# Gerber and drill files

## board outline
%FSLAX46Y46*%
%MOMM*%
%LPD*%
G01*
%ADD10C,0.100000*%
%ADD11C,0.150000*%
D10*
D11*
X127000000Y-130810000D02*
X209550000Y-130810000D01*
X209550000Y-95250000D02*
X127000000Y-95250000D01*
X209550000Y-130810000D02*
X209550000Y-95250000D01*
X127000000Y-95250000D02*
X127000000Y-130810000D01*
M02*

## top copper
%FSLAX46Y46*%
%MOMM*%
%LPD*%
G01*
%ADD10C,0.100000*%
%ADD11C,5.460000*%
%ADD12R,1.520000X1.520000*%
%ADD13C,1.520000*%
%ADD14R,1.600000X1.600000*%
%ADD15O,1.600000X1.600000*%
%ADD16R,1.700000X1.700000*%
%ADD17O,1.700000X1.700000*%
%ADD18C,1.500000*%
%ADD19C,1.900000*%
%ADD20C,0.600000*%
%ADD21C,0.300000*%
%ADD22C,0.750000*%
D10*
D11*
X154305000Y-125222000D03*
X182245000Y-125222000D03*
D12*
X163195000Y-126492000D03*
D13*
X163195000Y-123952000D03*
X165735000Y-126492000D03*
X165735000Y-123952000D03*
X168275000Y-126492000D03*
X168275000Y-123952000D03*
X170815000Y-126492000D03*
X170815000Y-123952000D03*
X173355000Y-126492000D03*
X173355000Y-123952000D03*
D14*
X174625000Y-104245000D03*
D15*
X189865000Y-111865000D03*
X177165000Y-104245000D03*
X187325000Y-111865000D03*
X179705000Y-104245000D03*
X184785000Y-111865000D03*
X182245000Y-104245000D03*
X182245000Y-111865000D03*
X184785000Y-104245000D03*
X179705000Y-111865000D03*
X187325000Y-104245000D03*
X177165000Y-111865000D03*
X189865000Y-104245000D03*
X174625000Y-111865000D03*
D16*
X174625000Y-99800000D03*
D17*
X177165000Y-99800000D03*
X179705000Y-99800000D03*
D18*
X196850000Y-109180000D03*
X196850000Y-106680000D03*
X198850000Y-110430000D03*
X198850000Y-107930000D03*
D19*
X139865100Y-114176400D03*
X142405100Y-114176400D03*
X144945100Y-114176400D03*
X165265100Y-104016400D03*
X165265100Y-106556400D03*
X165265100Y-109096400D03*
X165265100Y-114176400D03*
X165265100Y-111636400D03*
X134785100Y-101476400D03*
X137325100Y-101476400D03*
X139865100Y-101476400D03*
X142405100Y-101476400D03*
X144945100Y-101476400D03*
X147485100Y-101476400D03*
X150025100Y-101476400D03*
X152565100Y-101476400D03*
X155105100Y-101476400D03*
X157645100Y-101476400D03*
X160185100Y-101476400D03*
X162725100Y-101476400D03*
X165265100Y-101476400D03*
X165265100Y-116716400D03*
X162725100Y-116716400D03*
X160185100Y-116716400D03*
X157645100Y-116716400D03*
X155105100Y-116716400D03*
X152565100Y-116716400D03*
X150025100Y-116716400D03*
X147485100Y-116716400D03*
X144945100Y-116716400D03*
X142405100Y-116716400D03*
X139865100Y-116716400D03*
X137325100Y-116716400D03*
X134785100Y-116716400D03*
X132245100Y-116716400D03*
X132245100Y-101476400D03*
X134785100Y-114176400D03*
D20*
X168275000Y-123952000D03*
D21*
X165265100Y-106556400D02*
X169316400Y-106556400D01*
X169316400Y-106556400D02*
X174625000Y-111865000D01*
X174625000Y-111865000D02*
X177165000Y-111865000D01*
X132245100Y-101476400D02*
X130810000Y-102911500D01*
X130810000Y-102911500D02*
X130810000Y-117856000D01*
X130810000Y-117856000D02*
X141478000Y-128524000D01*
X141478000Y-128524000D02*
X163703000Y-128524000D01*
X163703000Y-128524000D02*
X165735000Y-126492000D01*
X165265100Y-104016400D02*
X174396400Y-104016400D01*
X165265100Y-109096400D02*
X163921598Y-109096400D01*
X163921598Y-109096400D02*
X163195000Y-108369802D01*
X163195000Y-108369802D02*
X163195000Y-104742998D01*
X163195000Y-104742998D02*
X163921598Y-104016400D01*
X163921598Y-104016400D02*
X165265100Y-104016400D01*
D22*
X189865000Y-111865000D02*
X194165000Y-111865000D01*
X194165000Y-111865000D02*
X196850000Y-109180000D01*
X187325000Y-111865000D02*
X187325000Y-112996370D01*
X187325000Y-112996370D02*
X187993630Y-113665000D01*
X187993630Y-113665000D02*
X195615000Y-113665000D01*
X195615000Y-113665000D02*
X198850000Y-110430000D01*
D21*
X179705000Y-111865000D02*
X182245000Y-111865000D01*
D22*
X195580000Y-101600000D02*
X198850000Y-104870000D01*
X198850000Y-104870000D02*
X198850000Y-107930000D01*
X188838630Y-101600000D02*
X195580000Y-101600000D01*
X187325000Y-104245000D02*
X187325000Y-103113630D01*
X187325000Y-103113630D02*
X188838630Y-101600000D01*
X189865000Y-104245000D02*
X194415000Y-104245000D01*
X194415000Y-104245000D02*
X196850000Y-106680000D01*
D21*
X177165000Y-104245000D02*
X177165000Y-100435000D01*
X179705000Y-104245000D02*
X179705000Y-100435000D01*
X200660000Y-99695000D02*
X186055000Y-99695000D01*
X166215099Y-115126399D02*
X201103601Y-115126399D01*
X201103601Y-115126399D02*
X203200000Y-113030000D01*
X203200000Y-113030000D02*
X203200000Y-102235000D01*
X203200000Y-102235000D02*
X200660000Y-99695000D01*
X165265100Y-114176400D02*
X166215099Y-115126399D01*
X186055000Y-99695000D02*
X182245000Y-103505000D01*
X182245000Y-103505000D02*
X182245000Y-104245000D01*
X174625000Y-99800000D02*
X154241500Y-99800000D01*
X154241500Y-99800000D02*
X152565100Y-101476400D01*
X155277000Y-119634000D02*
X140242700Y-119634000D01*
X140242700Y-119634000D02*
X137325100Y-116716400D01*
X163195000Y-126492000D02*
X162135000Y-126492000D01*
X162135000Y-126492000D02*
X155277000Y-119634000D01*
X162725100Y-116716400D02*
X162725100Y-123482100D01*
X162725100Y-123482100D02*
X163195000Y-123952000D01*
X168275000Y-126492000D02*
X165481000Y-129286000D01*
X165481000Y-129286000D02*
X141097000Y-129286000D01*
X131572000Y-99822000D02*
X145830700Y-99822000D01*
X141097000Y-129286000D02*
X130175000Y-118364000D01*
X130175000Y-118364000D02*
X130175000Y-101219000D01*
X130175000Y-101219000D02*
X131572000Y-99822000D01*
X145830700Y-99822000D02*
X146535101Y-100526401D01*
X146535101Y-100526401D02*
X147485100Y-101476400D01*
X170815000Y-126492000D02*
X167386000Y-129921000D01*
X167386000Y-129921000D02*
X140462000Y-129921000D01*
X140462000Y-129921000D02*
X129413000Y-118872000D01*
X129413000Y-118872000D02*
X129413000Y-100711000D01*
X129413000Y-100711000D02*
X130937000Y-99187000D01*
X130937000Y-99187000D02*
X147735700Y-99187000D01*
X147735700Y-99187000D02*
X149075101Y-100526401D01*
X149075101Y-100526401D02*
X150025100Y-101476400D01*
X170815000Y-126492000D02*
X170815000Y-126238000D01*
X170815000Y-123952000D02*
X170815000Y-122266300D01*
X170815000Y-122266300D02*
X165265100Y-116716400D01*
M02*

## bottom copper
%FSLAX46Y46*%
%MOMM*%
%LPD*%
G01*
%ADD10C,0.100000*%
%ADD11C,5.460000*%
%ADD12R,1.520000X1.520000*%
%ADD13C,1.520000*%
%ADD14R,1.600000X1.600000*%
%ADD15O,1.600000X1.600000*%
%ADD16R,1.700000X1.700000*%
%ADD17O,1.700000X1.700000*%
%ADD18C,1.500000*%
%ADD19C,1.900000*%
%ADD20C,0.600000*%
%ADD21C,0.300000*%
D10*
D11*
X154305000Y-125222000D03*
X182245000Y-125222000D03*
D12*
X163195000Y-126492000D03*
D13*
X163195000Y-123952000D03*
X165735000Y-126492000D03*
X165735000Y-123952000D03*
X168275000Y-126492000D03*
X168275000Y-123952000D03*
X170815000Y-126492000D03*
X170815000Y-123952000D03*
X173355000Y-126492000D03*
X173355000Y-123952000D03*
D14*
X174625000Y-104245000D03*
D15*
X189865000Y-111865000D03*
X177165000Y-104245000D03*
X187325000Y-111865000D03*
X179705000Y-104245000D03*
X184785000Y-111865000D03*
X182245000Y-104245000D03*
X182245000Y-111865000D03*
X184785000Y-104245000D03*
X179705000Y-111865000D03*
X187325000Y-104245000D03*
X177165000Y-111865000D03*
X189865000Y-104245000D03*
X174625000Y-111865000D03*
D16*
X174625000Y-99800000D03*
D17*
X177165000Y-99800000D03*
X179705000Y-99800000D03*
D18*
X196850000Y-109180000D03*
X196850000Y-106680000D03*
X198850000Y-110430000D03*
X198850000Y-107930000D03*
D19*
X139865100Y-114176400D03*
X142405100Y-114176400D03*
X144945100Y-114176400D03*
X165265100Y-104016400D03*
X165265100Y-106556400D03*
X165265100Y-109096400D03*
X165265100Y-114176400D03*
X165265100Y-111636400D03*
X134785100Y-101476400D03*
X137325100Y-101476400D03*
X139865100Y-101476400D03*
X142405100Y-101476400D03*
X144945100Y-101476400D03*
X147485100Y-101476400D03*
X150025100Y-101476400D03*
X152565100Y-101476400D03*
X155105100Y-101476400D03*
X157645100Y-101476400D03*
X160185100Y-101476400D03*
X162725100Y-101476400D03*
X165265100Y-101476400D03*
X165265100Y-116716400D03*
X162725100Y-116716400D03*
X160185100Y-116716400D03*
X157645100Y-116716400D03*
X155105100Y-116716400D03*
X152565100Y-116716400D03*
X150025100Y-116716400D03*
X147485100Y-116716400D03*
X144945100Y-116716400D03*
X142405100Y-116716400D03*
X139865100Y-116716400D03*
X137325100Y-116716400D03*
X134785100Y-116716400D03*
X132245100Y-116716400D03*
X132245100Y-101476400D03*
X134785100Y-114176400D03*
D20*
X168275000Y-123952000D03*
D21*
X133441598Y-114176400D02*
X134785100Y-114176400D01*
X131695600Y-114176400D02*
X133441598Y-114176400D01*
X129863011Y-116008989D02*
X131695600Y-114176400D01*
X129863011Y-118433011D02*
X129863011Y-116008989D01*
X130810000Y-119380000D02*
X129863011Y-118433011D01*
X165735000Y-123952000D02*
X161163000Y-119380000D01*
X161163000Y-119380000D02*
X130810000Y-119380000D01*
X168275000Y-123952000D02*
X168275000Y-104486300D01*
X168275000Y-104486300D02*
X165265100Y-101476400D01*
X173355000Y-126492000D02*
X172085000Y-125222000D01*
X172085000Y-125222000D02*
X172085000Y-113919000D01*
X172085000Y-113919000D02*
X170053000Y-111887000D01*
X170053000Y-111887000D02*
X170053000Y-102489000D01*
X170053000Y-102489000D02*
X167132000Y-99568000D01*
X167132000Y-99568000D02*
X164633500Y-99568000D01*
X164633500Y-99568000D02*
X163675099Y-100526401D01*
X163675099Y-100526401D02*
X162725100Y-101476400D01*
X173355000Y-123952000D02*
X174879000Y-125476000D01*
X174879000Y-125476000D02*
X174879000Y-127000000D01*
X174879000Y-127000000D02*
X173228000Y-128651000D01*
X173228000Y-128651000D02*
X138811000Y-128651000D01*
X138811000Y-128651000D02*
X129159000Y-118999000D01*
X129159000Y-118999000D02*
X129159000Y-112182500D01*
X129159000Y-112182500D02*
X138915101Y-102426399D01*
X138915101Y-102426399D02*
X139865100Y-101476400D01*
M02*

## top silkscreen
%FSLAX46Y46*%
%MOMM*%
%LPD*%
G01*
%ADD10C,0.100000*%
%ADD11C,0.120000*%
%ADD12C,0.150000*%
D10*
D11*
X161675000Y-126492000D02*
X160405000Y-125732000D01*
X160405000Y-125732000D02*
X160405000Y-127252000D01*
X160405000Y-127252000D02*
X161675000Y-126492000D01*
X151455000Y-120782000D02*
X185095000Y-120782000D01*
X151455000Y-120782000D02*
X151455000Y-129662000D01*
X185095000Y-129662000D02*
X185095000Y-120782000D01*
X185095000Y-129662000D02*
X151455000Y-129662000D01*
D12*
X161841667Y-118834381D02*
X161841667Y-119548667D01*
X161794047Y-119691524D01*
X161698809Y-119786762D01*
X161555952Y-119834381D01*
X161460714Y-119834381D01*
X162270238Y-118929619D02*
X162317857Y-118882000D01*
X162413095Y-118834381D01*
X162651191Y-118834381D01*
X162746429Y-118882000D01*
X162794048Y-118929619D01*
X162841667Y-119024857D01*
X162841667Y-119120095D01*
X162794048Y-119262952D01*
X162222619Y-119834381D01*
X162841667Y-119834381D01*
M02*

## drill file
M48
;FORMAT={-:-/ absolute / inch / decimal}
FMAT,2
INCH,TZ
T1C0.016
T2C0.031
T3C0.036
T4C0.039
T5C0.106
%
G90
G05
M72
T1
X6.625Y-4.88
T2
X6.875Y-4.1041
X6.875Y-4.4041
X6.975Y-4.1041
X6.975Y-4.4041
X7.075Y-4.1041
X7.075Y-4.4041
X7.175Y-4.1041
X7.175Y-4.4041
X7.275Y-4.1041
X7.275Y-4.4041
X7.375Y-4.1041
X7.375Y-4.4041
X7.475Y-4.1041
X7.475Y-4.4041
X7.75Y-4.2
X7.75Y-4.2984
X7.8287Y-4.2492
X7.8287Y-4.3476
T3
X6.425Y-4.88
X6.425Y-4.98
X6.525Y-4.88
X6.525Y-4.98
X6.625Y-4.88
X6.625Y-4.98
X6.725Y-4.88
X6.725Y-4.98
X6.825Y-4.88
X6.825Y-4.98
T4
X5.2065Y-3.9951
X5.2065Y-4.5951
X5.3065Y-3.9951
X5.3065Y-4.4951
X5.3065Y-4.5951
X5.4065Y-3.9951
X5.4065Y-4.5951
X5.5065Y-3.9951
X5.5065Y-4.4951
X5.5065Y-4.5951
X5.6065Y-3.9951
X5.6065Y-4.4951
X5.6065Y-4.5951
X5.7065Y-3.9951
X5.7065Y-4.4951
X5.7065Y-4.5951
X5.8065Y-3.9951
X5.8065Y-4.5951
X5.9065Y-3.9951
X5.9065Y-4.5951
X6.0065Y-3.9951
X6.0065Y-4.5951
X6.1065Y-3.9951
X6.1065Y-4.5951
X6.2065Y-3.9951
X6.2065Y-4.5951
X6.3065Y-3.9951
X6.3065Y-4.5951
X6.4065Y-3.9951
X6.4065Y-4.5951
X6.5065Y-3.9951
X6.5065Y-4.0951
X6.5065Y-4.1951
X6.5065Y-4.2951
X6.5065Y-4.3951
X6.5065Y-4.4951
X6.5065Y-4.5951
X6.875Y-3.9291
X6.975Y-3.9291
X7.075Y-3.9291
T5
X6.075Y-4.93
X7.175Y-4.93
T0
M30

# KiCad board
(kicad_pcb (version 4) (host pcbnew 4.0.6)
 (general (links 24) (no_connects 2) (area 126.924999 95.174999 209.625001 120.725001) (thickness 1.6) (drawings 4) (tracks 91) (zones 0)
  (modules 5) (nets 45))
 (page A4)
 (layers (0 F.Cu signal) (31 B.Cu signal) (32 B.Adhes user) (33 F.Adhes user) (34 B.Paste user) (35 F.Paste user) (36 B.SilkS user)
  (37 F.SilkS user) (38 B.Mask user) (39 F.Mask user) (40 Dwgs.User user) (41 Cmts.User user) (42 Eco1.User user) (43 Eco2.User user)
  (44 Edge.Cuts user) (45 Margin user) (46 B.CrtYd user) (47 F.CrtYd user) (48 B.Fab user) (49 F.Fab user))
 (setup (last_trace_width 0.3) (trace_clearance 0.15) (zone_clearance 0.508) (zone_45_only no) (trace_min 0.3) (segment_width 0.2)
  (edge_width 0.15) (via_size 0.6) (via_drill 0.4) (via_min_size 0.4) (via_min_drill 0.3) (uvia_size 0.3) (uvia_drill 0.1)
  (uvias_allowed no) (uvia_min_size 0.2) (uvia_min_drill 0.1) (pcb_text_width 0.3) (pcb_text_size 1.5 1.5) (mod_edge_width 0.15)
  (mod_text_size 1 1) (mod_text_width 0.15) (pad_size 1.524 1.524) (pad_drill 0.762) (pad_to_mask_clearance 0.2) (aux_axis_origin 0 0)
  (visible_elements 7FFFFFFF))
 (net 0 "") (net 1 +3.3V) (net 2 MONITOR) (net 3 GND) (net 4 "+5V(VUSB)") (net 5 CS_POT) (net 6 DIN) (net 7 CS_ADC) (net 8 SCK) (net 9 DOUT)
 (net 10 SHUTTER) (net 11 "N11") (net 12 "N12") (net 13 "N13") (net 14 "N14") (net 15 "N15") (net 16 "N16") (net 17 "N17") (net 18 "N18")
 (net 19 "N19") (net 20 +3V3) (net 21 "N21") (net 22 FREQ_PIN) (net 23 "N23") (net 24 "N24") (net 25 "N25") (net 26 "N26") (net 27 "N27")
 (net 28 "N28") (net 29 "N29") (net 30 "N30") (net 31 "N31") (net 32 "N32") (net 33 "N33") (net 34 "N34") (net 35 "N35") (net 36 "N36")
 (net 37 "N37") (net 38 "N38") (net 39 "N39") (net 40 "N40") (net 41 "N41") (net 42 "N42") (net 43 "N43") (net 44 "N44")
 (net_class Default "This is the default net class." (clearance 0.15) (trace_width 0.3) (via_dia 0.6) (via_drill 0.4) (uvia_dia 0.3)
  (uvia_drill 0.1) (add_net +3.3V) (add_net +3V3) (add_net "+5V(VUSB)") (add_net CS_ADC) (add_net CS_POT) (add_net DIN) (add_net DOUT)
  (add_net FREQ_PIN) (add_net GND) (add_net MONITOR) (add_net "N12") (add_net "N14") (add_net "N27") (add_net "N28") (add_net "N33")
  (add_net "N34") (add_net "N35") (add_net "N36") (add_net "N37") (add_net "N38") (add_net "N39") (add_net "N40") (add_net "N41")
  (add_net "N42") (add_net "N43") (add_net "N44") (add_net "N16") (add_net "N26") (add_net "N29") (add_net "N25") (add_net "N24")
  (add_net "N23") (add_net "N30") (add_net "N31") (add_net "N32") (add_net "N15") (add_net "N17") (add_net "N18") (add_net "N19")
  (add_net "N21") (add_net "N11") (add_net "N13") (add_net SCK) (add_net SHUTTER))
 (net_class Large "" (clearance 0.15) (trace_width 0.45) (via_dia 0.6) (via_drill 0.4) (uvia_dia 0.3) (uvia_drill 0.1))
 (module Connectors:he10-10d (layer F.Cu) (at 163.195 126.492)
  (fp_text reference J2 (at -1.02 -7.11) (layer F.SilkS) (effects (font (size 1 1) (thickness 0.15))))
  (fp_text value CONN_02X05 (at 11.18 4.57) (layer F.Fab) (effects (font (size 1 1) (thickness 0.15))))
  (fp_line (start -1.52 0) (end -2.79 -0.76) (layer F.SilkS) (width 0.12))
  (fp_line (start -2.79 -0.76) (end -2.79 0.76) (layer F.SilkS) (width 0.12))
  (fp_line (start -2.79 0.76) (end -1.52 0) (layer F.SilkS) (width 0.12))
  (fp_line (start -11.74 -5.71) (end 21.9 -5.71) (layer F.SilkS) (width 0.12))
  (fp_line (start -11.74 -5.71) (end -11.74 3.17) (layer F.SilkS) (width 0.12))
  (fp_line (start 21.9 3.17) (end 21.9 -5.71) (layer F.SilkS) (width 0.12))
  (fp_line (start 21.9 3.17) (end -11.74 3.17) (layer F.SilkS) (width 0.12))
  (pad "" thru_hole circle (at -8.89 -1.27) (size 5.46 5.46) (drill 2.69) (layers *.Cu *.Mask))
  (pad "" thru_hole circle (at 19.05 -1.27) (size 5.46 5.46) (drill 2.69) (layers *.Cu *.Mask))
  (pad 1 thru_hole rect (at 0 0) (size 1.52 1.52) (drill 0.91) (layers *.Cu *.Mask) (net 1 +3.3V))
  (pad 2 thru_hole circle (at 0 -2.54) (size 1.52 1.52) (drill 0.91) (layers *.Cu *.Mask) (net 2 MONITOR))
  (pad 3 thru_hole circle (at 2.54 0) (size 1.52 1.52) (drill 0.91) (layers *.Cu *.Mask) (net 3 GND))
  (pad 4 thru_hole circle (at 2.54 -2.54) (size 1.52 1.52) (drill 0.91) (layers *.Cu *.Mask) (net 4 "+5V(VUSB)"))
  (pad 5 thru_hole circle (at 5.08 0) (size 1.52 1.52) (drill 0.91) (layers *.Cu *.Mask) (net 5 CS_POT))
  (pad 6 thru_hole circle (at 5.08 -2.54) (size 1.52 1.52) (drill 0.91) (layers *.Cu *.Mask) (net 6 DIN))
  (pad 7 thru_hole circle (at 7.62 0) (size 1.52 1.52) (drill 0.91) (layers *.Cu *.Mask) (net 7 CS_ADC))
  (pad 8 thru_hole circle (at 7.62 -2.54) (size 1.52 1.52) (drill 0.91) (layers *.Cu *.Mask) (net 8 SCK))
  (pad 9 thru_hole circle (at 10.16 0) (size 1.52 1.52) (drill 0.91) (layers *.Cu *.Mask) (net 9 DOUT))
  (pad 10 thru_hole circle (at 10.16 -2.54) (size 1.52 1.52) (drill 0.91) (layers *.Cu *.Mask) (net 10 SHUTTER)))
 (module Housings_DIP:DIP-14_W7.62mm (layer B.Cu) (at 174.625 104.245 270)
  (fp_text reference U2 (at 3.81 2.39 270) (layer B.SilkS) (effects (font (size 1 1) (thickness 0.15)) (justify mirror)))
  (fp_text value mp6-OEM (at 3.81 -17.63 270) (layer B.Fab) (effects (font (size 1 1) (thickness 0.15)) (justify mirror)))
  (pad 1 thru_hole rect (at 0 0 270) (size 1.6 1.6) (drill 0.8) (layers *.Cu *.Mask) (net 3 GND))
  (pad 8 thru_hole oval (at 7.62 -15.24 270) (size 1.6 1.6) (drill 0.8) (layers *.Cu *.Mask) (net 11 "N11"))
  (pad 2 thru_hole oval (at 0 -2.54 270) (size 1.6 1.6) (drill 0.8) (layers *.Cu *.Mask) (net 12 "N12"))
  (pad 9 thru_hole oval (at 7.62 -12.7 270) (size 1.6 1.6) (drill 0.8) (layers *.Cu *.Mask) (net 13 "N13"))
  (pad 3 thru_hole oval (at 0 -5.08 270) (size 1.6 1.6) (drill 0.8) (layers *.Cu *.Mask) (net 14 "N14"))
  (pad 10 thru_hole oval (at 7.62 -10.16 270) (size 1.6 1.6) (drill 0.8) (layers *.Cu *.Mask) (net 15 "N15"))
  (pad 4 thru_hole oval (at 0 -7.62 270) (size 1.6 1.6) (drill 0.8) (layers *.Cu *.Mask) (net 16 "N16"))
  (pad 11 thru_hole oval (at 7.62 -7.62 270) (size 1.6 1.6) (drill 0.8) (layers *.Cu *.Mask) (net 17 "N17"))
  (pad 5 thru_hole oval (at 0 -10.16 270) (size 1.6 1.6) (drill 0.8) (layers *.Cu *.Mask) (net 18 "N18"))
  (pad 12 thru_hole oval (at 7.62 -5.08 270) (size 1.6 1.6) (drill 0.8) (layers *.Cu *.Mask) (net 17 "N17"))
  (pad 6 thru_hole oval (at 0 -12.7 270) (size 1.6 1.6) (drill 0.8) (layers *.Cu *.Mask) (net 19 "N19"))
  (pad 13 thru_hole oval (at 7.62 -2.54 270) (size 1.6 1.6) (drill 0.8) (layers *.Cu *.Mask) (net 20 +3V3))
  (pad 7 thru_hole oval (at 0 -15.24 270) (size 1.6 1.6) (drill 0.8) (layers *.Cu *.Mask) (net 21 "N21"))
  (pad 14 thru_hole oval (at 7.62 0 270) (size 1.6 1.6) (drill 0.8) (layers *.Cu *.Mask) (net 20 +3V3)))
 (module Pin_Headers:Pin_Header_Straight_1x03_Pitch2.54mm (layer B.Cu) (at 174.625 99.8 270)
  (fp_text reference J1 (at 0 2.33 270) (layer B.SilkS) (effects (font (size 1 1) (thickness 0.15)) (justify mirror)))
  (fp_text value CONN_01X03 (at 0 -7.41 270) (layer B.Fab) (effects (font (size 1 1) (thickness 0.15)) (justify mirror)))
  (pad 1 thru_hole rect (at 0 0 270) (size 1.7 1.7) (drill 1) (layers *.Cu *.Mask) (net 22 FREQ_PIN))
  (pad 2 thru_hole oval (at 0 -2.54 270) (size 1.7 1.7) (drill 1) (layers *.Cu *.Mask) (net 12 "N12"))
  (pad 3 thru_hole oval (at 0 -5.08 270) (size 1.7 1.7) (drill 1) (layers *.Cu *.Mask) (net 14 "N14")))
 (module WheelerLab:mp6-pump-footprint (layer B.Cu) (at 197.85 108.43)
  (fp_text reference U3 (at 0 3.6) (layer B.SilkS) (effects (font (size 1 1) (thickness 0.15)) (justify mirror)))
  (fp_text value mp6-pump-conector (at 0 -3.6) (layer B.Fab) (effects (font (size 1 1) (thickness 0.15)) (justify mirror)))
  (pad 2 thru_hole circle (at -1 0.75) (size 1.5 1.5) (drill 0.8) (layers *.Cu *.Mask) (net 11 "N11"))
  (pad 4 thru_hole circle (at -1 -1.75) (size 1.5 1.5) (drill 0.8) (layers *.Cu *.Mask) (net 21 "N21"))
  (pad 1 thru_hole circle (at 1 2) (size 1.5 1.5) (drill 0.8) (layers *.Cu *.Mask) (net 13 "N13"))
  (pad 3 thru_hole circle (at 1 -0.5) (size 1.5 1.5) (drill 0.8) (layers *.Cu *.Mask) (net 19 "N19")))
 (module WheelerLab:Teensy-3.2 (layer B.Cu) (at 148.5011 109.0964)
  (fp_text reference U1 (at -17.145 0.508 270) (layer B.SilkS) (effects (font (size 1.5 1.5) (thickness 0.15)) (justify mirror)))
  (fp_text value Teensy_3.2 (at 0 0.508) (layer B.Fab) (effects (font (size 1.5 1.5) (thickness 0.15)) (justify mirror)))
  (pad 35 thru_hole circle (at -8.636 5.08) (size 1.9 1.9) (drill 1) (layers *.Cu *.Mask B.SilkS) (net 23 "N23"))
  (pad 34 thru_hole circle (at -6.096 5.08) (size 1.9 1.9) (drill 1) (layers *.Cu *.Mask B.SilkS) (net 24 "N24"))
  (pad 33 thru_hole circle (at -3.556 5.08) (size 1.9 1.9) (drill 1) (layers *.Cu *.Mask B.SilkS) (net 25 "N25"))
  (pad 32 thru_hole circle (at 16.764 -5.08) (size 1.9 1.9) (drill 1) (layers *.Cu *.Mask B.SilkS) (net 3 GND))
  (pad 31 thru_hole circle (at 16.764 -2.54) (size 1.9 1.9) (drill 1) (layers *.Cu *.Mask B.SilkS) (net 20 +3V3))
  (pad 30 thru_hole circle (at 16.764 0) (size 1.9 1.9) (drill 1) (layers *.Cu *.Mask B.SilkS) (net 3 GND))
  (pad 28 thru_hole circle (at 16.764 5.08) (size 1.9 1.9) (drill 1) (layers *.Cu *.Mask B.SilkS) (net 16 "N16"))
  (pad 29 thru_hole circle (at 16.764 2.54) (size 1.9 1.9) (drill 1) (layers *.Cu *.Mask B.SilkS) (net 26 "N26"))
  (pad 0 thru_hole circle (at -13.716 -7.62) (size 1.9 1.9) (drill 1) (layers *.Cu *.Mask B.SilkS) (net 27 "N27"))
  (pad 1 thru_hole circle (at -11.176 -7.62) (size 1.9 1.9) (drill 1) (layers *.Cu *.Mask B.SilkS) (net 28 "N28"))
  (pad 2 thru_hole circle (at -8.636 -7.62) (size 1.9 1.9) (drill 1) (layers *.Cu *.Mask B.SilkS) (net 10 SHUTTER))
  (pad 3 thru_hole circle (at -6.096 -7.62) (size 1.9 1.9) (drill 1) (layers *.Cu *.Mask B.SilkS) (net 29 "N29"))
  (pad 4 thru_hole circle (at -3.556 -7.62) (size 1.9 1.9) (drill 1) (layers *.Cu *.Mask B.SilkS) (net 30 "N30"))
  (pad 5 thru_hole circle (at -1.016 -7.62) (size 1.9 1.9) (drill 1) (layers *.Cu *.Mask B.SilkS) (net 5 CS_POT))
  (pad 6 thru_hole circle (at 1.524 -7.62) (size 1.9 1.9) (drill 1) (layers *.Cu *.Mask B.SilkS) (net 7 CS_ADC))
  (pad 7 thru_hole circle (at 4.064 -7.62) (size 1.9 1.9) (drill 1) (layers *.Cu *.Mask B.SilkS) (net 22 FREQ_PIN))
  (pad 8 thru_hole circle (at 6.604 -7.62) (size 1.9 1.9) (drill 1) (layers *.Cu *.Mask B.SilkS) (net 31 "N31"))
  (pad 9 thru_hole circle (at 9.144 -7.62) (size 1.9 1.9) (drill 1) (layers *.Cu *.Mask B.SilkS) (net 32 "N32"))
  (pad 10 thru_hole circle (at 11.684 -7.62) (size 1.9 1.9) (drill 1) (layers *.Cu *.Mask B.SilkS) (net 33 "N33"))
  (pad 11 thru_hole circle (at 14.224 -7.62) (size 1.9 1.9) (drill 1) (layers *.Cu *.Mask B.SilkS) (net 9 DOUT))
  (pad 12 thru_hole circle (at 16.764 -7.62) (size 1.9 1.9) (drill 1) (layers *.Cu *.Mask B.SilkS) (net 6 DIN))
  (pad 13 thru_hole circle (at 16.764 7.62) (size 1.9 1.9) (drill 1) (layers *.Cu *.Mask B.SilkS) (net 8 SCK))
  (pad 14 thru_hole circle (at 14.224 7.62) (size 1.9 1.9) (drill 1) (layers *.Cu *.Mask B.SilkS) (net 2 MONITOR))
  (pad 15 thru_hole circle (at 11.684 7.62) (size 1.9 1.9) (drill 1) (layers *.Cu *.Mask B.SilkS) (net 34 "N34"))
  (pad 16 thru_hole circle (at 9.144 7.62) (size 1.9 1.9) (drill 1) (layers *.Cu *.Mask B.SilkS) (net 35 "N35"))
  (pad 17 thru_hole circle (at 6.604 7.62) (size 1.9 1.9) (drill 1) (layers *.Cu *.Mask B.SilkS) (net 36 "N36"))
  (pad 18 thru_hole circle (at 4.064 7.62) (size 1.9 1.9) (drill 1) (layers *.Cu *.Mask B.SilkS) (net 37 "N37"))
  (pad 19 thru_hole circle (at 1.524 7.62) (size 1.9 1.9) (drill 1) (layers *.Cu *.Mask B.SilkS) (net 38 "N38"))
  (pad 20 thru_hole circle (at -1.016 7.62) (size 1.9 1.9) (drill 1) (layers *.Cu *.Mask B.SilkS) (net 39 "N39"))
  (pad 21 thru_hole circle (at -3.556 7.62) (size 1.9 1.9) (drill 1) (layers *.Cu *.Mask B.SilkS) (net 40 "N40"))
  (pad 22 thru_hole circle (at -6.096 7.62) (size 1.9 1.9) (drill 1) (layers *.Cu *.Mask B.SilkS) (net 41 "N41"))
  (pad 23 thru_hole circle (at -8.636 7.62) (size 1.9 1.9) (drill 1) (layers *.Cu *.Mask B.SilkS) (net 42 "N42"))
  (pad 24 thru_hole circle (at -11.176 7.62) (size 1.9 1.9) (drill 1) (layers *.Cu *.Mask B.SilkS) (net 1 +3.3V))
  (pad 25 thru_hole circle (at -13.716 7.62) (size 1.9 1.9) (drill 1) (layers *.Cu *.Mask B.SilkS) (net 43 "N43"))
  (pad 26 thru_hole circle (at -16.256 7.62) (size 1.9 1.9) (drill 1) (layers *.Cu *.Mask B.SilkS) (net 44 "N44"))
  (pad 27 thru_hole circle (at -16.256 -7.62) (size 1.9 1.9) (drill 1) (layers *.Cu *.Mask B.SilkS) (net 3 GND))
  (pad 36 thru_hole circle (at -13.716 5.08) (size 1.9 1.9) (drill 1) (layers *.Cu *.Mask B.SilkS) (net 4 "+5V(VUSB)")))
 (gr_line (start 127 130.81) (end 209.55 130.81) (layer Edge.Cuts) (width 0.15))
 (gr_line (start 209.55 95.25) (end 127 95.25) (layer Edge.Cuts) (width 0.15))
 (gr_line (start 209.55 130.81) (end 209.55 95.25) (layer Edge.Cuts) (width 0.15))
 (gr_line (start 127 95.25) (end 127 130.81) (layer Edge.Cuts) (width 0.15))
 (segment (start 165.2651 106.5564) (end 169.3164 106.5564) (width 0.3) (layer F.Cu) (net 20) (status 10))
 (segment (start 169.3164 106.5564) (end 174.625 111.865) (width 0.3) (layer F.Cu) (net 20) (status 20))
 (segment (start 174.625 111.865) (end 177.165 111.865) (width 0.3) (layer F.Cu) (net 20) (status 30))
 (segment (start 132.2451 101.4764) (end 130.81 102.9115) (width 0.3) (layer F.Cu) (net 3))
 (segment (start 130.81 102.9115) (end 130.81 117.856) (width 0.3) (layer F.Cu) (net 3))
 (segment (start 130.81 117.856) (end 141.478 128.524) (width 0.3) (layer F.Cu) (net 3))
 (segment (start 141.478 128.524) (end 163.703 128.524) (width 0.3) (layer F.Cu) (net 3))
 (segment (start 163.703 128.524) (end 165.735 126.492) (width 0.3) (layer F.Cu) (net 3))
 (segment (start 165.2651 104.0164) (end 174.3964 104.0164) (width 0.3) (layer F.Cu) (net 3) (status 30))
 (segment (start 165.2651 109.0964) (end 163.921598 109.0964) (width 0.3) (layer F.Cu) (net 3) (status 10))
 (segment (start 163.921598 109.0964) (end 163.195 108.369802) (width 0.3) (layer F.Cu) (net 3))
 (segment (start 163.195 108.369802) (end 163.195 104.742998) (width 0.3) (layer F.Cu) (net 3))
 (segment (start 163.195 104.742998) (end 163.921598 104.0164) (width 0.3) (layer F.Cu) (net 3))
 (segment (start 163.921598 104.0164) (end 165.2651 104.0164) (width 0.3) (layer F.Cu) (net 3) (status 20))
 (segment (start 189.865 111.865) (end 194.165 111.865) (width 0.75) (layer F.Cu) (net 11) (status 10))
 (segment (start 194.165 111.865) (end 196.85 109.18) (width 0.75) (layer F.Cu) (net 11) (status 20))
 (segment (start 187.325 111.865) (end 187.325 112.99637) (width 0.75) (layer F.Cu) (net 13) (status 10))
 (segment (start 187.325 112.99637) (end 187.99363 113.665) (width 0.75) (layer F.Cu) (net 13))
 (segment (start 187.99363 113.665) (end 195.615 113.665) (width 0.75) (layer F.Cu) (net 13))
 (segment (start 195.615 113.665) (end 198.85 110.43) (width 0.75) (layer F.Cu) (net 13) (status 20))
 (segment (start 179.705 111.865) (end 182.245 111.865) (width 0.3) (layer F.Cu) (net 17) (status 30))
 (segment (start 195.58 101.6) (end 198.85 104.87) (width 0.75) (layer F.Cu) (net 19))
 (segment (start 198.85 104.87) (end 198.85 107.93) (width 0.75) (layer F.Cu) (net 19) (status 20))
 (segment (start 188.83863 101.6) (end 195.58 101.6) (width 0.75) (layer F.Cu) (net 19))
 (segment (start 187.325 104.245) (end 187.325 103.11363) (width 0.75) (layer F.Cu) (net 19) (status 10))
 (segment (start 187.325 103.11363) (end 188.83863 101.6) (width 0.75) (layer F.Cu) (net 19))
 (segment (start 189.865 104.245) (end 194.415 104.245) (width 0.75) (layer F.Cu) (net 21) (status 10))
 (segment (start 194.415 104.245) (end 196.85 106.68) (width 0.75) (layer F.Cu) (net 21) (status 20))
 (segment (start 177.165 104.245) (end 177.165 100.435) (width 0.3) (layer F.Cu) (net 12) (status 30))
 (segment (start 179.705 104.245) (end 179.705 100.435) (width 0.3) (layer F.Cu) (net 14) (status 30))
 (segment (start 200.66 99.695) (end 186.055 99.695) (width 0.3) (layer F.Cu) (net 16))
 (segment (start 166.215099 115.126399) (end 201.103601 115.126399) (width 0.3) (layer F.Cu) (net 16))
 (segment (start 201.103601 115.126399) (end 203.2 113.03) (width 0.3) (layer F.Cu) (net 16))
 (segment (start 203.2 113.03) (end 203.2 102.235) (width 0.3) (layer F.Cu) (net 16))
 (segment (start 203.2 102.235) (end 200.66 99.695) (width 0.3) (layer F.Cu) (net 16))
 (segment (start 165.2651 114.1764) (end 166.215099 115.126399) (width 0.3) (layer F.Cu) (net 16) (status 10))
 (segment (start 186.055 99.695) (end 182.245 103.505) (width 0.3) (layer F.Cu) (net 16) (status 20))
 (segment (start 182.245 103.505) (end 182.245 104.245) (width 0.3) (layer F.Cu) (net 16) (status 30))
 (segment (start 174.625 99.8) (end 154.2415 99.8) (width 0.3) (layer F.Cu) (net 22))
 (segment (start 154.2415 99.8) (end 152.5651 101.4764) (width 0.3) (layer F.Cu) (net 22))
 (segment (start 155.277 119.634) (end 140.2427 119.634) (width 0.3) (layer F.Cu) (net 1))
 (segment (start 140.2427 119.634) (end 137.3251 116.7164) (width 0.3) (layer F.Cu) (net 1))
 (segment (start 163.195 126.492) (end 162.135 126.492) (width 0.3) (layer F.Cu) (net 1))
 (segment (start 162.135 126.492) (end 155.277 119.634) (width 0.3) (layer F.Cu) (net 1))
 (segment (start 162.7251 116.7164) (end 162.7251 123.4821) (width 0.3) (layer F.Cu) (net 2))
 (segment (start 162.7251 123.4821) (end 163.195 123.952) (width 0.3) (layer F.Cu) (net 2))
 (segment (start 133.441598 114.1764) (end 134.7851 114.1764) (width 0.3) (layer B.Cu) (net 4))
 (segment (start 131.6956 114.1764) (end 133.441598 114.1764) (width 0.3) (layer B.Cu) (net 4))
 (segment (start 129.863011 116.008989) (end 131.6956 114.1764) (width 0.3) (layer B.Cu) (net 4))
 (segment (start 129.863011 118.433011) (end 129.863011 116.008989) (width 0.3) (layer B.Cu) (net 4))
 (segment (start 130.81 119.38) (end 129.863011 118.433011) (width 0.3) (layer B.Cu) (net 4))
 (segment (start 165.735 123.952) (end 161.163 119.38) (width 0.3) (layer B.Cu) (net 4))
 (segment (start 161.163 119.38) (end 130.81 119.38) (width 0.3) (layer B.Cu) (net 4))
 (segment (start 168.275 126.492) (end 165.481 129.286) (width 0.3) (layer F.Cu) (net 5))
 (segment (start 165.481 129.286) (end 141.097 129.286) (width 0.3) (layer F.Cu) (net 5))
 (segment (start 131.572 99.822) (end 145.8307 99.822) (width 0.3) (layer F.Cu) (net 5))
 (segment (start 141.097 129.286) (end 130.175 118.364) (width 0.3) (layer F.Cu) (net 5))
 (segment (start 130.175 118.364) (end 130.175 101.219) (width 0.3) (layer F.Cu) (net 5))
 (segment (start 130.175 101.219) (end 131.572 99.822) (width 0.3) (layer F.Cu) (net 5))
 (segment (start 145.8307 99.822) (end 146.535101 100.526401) (width 0.3) (layer F.Cu) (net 5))
 (segment (start 146.535101 100.526401) (end 147.4851 101.4764) (width 0.3) (layer F.Cu) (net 5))
 (segment (start 168.275 123.952) (end 168.275 104.4863) (width 0.3) (layer B.Cu) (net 6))
 (segment (start 168.275 104.4863) (end 165.2651 101.4764) (width 0.3) (layer B.Cu) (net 6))
 (via (at 168.275 123.952) (size 0.6) (drill 0.4) (layers F.Cu B.Cu) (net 6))
 (segment (start 170.815 126.492) (end 167.386 129.921) (width 0.3) (layer F.Cu) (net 7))
 (segment (start 167.386 129.921) (end 140.462 129.921) (width 0.3) (layer F.Cu) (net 7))
 (segment (start 140.462 129.921) (end 129.413 118.872) (width 0.3) (layer F.Cu) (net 7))
 (segment (start 129.413 118.872) (end 129.413 100.711) (width 0.3) (layer F.Cu) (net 7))
 (segment (start 129.413 100.711) (end 130.937 99.187) (width 0.3) (layer F.Cu) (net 7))
 (segment (start 130.937 99.187) (end 147.7357 99.187) (width 0.3) (layer F.Cu) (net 7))
 (segment (start 147.7357 99.187) (end 149.075101 100.526401) (width 0.3) (layer F.Cu) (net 7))
 (segment (start 149.075101 100.526401) (end 150.0251 101.4764) (width 0.3) (layer F.Cu) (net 7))
 (segment (start 170.815 126.492) (end 170.815 126.238) (width 0.3) (layer F.Cu) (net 7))
 (segment (start 170.815 123.952) (end 170.815 122.2663) (width 0.3) (layer F.Cu) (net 8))
 (segment (start 170.815 122.2663) (end 165.2651 116.7164) (width 0.3) (layer F.Cu) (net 8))
 (segment (start 173.355 126.492) (end 172.085 125.222) (width 0.3) (layer B.Cu) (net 9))
 (segment (start 172.085 125.222) (end 172.085 113.919) (width 0.3) (layer B.Cu) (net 9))
 (segment (start 172.085 113.919) (end 170.053 111.887) (width 0.3) (layer B.Cu) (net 9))
 (segment (start 170.053 111.887) (end 170.053 102.489) (width 0.3) (layer B.Cu) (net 9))
 (segment (start 170.053 102.489) (end 167.132 99.568) (width 0.3) (layer B.Cu) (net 9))
 (segment (start 167.132 99.568) (end 164.6335 99.568) (width 0.3) (layer B.Cu) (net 9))
 (segment (start 164.6335 99.568) (end 163.675099 100.526401) (width 0.3) (layer B.Cu) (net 9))
 (segment (start 163.675099 100.526401) (end 162.7251 101.4764) (width 0.3) (layer B.Cu) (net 9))
 (segment (start 173.355 123.952) (end 174.879 125.476) (width 0.3) (layer B.Cu) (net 10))
 (segment (start 174.879 125.476) (end 174.879 127) (width 0.3) (layer B.Cu) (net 10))
 (segment (start 174.879 127) (end 173.228 128.651) (width 0.3) (layer B.Cu) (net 10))
 (segment (start 173.228 128.651) (end 138.811 128.651) (width 0.3) (layer B.Cu) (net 10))
 (segment (start 138.811 128.651) (end 129.159 118.999) (width 0.3) (layer B.Cu) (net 10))
 (segment (start 129.159 118.999) (end 129.159 112.1825) (width 0.3) (layer B.Cu) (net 10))
 (segment (start 129.159 112.1825) (end 138.915101 102.426399) (width 0.3) (layer B.Cu) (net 10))
 (segment (start 138.915101 102.426399) (end 139.8651 101.4764) (width 0.3) (layer B.Cu) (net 10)))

